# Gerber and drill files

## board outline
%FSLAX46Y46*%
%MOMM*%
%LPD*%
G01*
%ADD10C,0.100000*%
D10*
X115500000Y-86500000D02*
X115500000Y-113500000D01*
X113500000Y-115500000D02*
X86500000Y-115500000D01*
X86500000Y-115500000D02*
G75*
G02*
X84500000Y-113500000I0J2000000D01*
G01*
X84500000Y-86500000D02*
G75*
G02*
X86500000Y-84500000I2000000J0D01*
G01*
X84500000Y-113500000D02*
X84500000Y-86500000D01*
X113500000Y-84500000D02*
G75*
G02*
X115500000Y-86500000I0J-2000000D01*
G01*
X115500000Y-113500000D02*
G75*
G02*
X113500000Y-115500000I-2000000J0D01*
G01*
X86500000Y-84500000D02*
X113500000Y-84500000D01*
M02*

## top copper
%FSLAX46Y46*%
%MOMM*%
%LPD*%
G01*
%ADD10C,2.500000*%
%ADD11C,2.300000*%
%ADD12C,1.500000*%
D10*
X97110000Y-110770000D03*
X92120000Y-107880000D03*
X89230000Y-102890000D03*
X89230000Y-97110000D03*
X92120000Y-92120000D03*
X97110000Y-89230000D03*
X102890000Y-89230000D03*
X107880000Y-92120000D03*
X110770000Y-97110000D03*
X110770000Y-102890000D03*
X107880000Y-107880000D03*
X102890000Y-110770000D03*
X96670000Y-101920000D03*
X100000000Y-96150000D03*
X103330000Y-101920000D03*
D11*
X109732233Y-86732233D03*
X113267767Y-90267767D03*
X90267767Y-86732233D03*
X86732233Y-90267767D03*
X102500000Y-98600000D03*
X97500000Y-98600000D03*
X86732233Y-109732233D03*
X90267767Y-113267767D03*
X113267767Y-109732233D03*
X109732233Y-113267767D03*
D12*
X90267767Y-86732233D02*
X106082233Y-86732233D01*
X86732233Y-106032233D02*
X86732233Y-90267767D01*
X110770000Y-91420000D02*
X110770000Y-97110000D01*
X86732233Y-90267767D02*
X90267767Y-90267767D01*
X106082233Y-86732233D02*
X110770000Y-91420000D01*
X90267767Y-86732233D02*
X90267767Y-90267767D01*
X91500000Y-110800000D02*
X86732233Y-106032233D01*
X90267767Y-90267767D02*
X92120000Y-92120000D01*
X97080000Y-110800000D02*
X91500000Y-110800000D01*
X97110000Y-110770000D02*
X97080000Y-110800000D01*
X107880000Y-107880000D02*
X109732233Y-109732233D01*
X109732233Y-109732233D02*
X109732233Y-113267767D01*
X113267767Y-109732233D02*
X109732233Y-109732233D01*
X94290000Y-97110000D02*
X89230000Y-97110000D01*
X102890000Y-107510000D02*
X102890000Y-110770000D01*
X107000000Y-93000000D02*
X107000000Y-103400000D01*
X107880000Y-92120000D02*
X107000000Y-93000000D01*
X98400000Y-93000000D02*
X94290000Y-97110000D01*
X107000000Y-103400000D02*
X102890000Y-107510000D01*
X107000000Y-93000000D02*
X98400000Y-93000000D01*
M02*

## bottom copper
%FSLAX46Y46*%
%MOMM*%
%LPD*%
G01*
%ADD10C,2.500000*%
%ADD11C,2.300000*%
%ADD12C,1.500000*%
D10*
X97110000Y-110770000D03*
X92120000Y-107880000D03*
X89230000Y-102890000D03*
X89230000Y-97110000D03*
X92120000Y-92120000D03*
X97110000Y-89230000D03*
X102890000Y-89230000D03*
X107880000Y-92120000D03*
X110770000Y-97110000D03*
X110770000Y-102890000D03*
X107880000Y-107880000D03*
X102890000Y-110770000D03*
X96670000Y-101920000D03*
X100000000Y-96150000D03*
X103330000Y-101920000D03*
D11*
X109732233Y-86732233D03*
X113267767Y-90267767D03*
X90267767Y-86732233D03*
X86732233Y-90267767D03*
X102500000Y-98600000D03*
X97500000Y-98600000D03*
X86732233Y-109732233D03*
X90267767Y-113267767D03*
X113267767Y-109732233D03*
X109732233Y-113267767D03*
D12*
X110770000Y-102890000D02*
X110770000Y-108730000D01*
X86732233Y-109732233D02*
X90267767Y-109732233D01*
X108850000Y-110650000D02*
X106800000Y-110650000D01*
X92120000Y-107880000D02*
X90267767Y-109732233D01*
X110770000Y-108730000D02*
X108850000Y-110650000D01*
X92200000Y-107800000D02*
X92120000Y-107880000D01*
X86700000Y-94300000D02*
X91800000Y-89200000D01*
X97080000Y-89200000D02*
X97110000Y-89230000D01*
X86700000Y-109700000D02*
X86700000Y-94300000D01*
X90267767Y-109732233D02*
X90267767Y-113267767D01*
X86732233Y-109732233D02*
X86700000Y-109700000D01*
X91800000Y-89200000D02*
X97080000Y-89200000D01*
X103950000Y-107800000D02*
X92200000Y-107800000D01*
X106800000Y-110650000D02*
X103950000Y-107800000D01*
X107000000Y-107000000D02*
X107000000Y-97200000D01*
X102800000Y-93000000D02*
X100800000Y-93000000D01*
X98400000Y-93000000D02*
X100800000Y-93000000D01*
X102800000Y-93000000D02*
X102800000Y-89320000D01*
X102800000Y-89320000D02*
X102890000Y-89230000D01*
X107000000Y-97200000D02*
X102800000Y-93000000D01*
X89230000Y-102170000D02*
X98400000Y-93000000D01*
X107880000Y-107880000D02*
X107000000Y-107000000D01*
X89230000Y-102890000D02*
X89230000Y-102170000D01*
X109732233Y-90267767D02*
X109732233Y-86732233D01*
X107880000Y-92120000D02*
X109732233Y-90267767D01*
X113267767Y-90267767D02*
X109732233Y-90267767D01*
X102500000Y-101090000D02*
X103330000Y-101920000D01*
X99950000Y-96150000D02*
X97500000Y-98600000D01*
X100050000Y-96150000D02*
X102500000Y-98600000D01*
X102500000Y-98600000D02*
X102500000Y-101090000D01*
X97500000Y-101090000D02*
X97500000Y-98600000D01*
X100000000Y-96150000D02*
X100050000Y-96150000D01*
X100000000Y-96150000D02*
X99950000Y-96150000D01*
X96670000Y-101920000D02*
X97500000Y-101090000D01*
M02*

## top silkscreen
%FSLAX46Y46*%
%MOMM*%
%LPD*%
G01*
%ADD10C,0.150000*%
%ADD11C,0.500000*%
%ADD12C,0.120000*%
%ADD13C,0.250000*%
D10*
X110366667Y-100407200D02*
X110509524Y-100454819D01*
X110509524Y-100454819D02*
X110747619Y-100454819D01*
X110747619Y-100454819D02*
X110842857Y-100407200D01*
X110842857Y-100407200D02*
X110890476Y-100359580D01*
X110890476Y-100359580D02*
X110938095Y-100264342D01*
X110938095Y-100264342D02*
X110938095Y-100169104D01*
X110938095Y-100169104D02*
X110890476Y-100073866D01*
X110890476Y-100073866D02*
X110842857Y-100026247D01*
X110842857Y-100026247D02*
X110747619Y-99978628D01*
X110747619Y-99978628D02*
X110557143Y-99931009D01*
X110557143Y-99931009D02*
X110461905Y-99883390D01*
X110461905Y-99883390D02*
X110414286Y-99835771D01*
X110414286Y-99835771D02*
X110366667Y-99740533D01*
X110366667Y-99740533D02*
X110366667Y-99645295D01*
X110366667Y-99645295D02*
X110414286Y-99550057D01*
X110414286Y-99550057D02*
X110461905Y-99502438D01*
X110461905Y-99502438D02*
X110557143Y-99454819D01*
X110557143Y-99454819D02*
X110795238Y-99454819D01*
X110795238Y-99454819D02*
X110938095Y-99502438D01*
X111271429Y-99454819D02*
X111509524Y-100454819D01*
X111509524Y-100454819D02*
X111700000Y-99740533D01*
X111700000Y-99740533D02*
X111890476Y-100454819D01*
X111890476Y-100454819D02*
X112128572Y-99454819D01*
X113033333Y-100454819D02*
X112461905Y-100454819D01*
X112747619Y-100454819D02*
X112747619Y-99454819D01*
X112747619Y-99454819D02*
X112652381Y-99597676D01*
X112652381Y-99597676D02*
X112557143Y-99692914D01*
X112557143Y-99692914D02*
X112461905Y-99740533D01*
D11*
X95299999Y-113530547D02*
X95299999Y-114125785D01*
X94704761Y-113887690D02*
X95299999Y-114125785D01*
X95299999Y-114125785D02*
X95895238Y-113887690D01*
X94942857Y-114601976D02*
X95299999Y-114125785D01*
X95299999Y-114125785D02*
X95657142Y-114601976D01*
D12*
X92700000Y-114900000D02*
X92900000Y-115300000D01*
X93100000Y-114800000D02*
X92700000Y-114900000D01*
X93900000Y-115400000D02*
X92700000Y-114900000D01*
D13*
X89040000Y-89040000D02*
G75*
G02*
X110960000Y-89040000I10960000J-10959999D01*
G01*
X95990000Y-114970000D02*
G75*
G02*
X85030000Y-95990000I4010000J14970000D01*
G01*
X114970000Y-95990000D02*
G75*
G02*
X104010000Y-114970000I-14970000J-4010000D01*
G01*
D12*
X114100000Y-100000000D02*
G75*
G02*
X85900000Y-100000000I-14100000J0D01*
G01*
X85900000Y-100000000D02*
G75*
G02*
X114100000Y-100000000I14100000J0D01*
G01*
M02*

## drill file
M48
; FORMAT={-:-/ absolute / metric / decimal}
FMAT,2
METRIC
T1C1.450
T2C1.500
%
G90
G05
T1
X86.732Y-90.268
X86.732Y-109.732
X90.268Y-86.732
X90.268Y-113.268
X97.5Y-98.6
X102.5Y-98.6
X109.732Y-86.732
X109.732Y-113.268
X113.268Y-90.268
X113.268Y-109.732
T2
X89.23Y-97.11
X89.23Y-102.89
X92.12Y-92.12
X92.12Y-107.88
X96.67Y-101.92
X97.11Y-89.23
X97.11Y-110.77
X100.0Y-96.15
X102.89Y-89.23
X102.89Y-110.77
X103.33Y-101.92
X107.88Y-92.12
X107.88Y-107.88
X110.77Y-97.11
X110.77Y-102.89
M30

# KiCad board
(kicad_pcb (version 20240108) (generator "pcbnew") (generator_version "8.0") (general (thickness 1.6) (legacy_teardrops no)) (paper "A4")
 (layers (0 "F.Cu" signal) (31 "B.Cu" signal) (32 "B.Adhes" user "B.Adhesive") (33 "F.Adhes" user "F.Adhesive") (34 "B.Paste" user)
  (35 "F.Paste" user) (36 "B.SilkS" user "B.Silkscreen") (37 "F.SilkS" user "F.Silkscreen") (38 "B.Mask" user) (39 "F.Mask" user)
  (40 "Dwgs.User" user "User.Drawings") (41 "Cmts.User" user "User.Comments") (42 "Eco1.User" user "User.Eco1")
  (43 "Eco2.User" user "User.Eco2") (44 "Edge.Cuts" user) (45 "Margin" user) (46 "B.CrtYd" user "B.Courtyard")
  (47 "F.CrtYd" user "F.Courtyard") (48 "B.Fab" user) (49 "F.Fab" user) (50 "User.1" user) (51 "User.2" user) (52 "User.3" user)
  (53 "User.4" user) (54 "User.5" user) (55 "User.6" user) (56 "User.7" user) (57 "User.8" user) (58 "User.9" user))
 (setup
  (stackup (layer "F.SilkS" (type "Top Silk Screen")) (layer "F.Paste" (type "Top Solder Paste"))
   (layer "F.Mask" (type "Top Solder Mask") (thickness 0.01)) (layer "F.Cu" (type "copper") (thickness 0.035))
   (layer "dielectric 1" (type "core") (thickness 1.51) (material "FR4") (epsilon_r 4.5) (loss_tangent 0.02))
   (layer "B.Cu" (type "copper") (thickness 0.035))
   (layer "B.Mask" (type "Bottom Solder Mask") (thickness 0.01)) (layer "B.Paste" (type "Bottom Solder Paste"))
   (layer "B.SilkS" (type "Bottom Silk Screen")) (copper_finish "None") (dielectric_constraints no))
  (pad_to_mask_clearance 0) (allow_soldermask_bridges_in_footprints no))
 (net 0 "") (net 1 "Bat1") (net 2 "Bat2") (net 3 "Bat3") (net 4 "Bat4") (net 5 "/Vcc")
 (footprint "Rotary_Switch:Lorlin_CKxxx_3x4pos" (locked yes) (layer "F.Cu") (at 100 100)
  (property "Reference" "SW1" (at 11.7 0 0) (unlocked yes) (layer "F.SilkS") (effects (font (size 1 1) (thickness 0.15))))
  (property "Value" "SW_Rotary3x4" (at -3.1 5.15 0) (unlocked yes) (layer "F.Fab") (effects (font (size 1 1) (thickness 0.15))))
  (fp_line (start -7.3 14.9) (end -7.1 15.3) (stroke (width 0.12) (type solid)) (layer "F.SilkS"))
  (fp_line (start -6.9 14.8) (end -7.3 14.9) (stroke (width 0.12) (type solid)) (layer "F.SilkS"))
  (fp_line (start -6.1 15.4) (end -7.3 14.9) (stroke (width 0.12) (type solid)) (layer "F.SilkS"))
  (fp_arc (start -10.96 -10.96) (mid 0 -15.499781) (end 10.96 -10.96) (stroke (width 0.25) (type solid)) (layer "F.SilkS"))
  (fp_arc (start -4.01 14.97) (mid -13.420887 7.74989) (end -14.97 -4.01) (stroke (width 0.25) (type solid)) (layer "F.SilkS"))
  (fp_arc (start 14.97 -4.01) (mid 13.420887 7.74989) (end 4.01 14.97) (stroke (width 0.25) (type solid)) (layer "F.SilkS"))
  (fp_circle (center 0 0) (end 14.1 0) (stroke (width 0.12) (type solid)) (fill none) (layer "F.SilkS"))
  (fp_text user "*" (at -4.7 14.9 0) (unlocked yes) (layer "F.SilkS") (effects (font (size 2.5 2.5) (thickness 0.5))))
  (pad "1" thru_hole circle (at -2.89 10.77) (size 2.5 2.5) (drill 1.5) (layers "*.Cu" "*.Mask") (remove_unused_layers no) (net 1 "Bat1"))
  (pad "2" thru_hole circle (at -7.88 7.88) (size 2.5 2.5) (drill 1.5) (layers "*.Cu" "*.Mask") (remove_unused_layers no) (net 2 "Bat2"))
  (pad "3" thru_hole circle (at -10.77 2.89) (size 2.5 2.5) (drill 1.5) (layers "*.Cu" "*.Mask") (remove_unused_layers no) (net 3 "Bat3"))
  (pad "4" thru_hole circle (at -10.77 -2.89) (size 2.5 2.5) (drill 1.5) (layers "*.Cu" "*.Mask") (remove_unused_layers no) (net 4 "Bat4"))
  (pad "5" thru_hole circle (at -7.88 -7.88) (size 2.5 2.5) (drill 1.5) (layers "*.Cu" "*.Mask") (remove_unused_layers no) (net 1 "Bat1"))
  (pad "6" thru_hole circle (at -2.89 -10.77) (size 2.5 2.5) (drill 1.5) (layers "*.Cu" "*.Mask") (remove_unused_layers no) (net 2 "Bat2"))
  (pad "7" thru_hole circle (at 2.89 -10.77) (size 2.5 2.5) (drill 1.5) (layers "*.Cu" "*.Mask") (remove_unused_layers no) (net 3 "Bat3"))
  (pad "8" thru_hole circle (at 7.88 -7.88) (size 2.5 2.5) (drill 1.5) (layers "*.Cu" "*.Mask") (remove_unused_layers no) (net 4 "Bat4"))
  (pad "9" thru_hole circle (at 10.77 -2.89) (size 2.5 2.5) (drill 1.5) (layers "*.Cu" "*.Mask") (remove_unused_layers no) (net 1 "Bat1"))
  (pad "10" thru_hole circle (at 10.77 2.89) (size 2.5 2.5) (drill 1.5) (layers "*.Cu" "*.Mask") (remove_unused_layers no) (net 2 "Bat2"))
  (pad "11" thru_hole circle (at 7.88 7.88) (size 2.5 2.5) (drill 1.5) (layers "*.Cu" "*.Mask") (remove_unused_layers no) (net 3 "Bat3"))
  (pad "12" thru_hole circle (at 2.89 10.77) (size 2.5 2.5) (drill 1.5) (layers "*.Cu" "*.Mask") (remove_unused_layers no) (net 4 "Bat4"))
  (pad "13" thru_hole circle (at -3.33 1.92) (size 2.5 2.5) (drill 1.5) (layers "*.Cu" "*.Mask") (remove_unused_layers no) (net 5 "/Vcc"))
  (pad "14" thru_hole circle (at 0 -3.85) (size 2.5 2.5) (drill 1.5) (layers "*.Cu" "*.Mask") (remove_unused_layers no) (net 5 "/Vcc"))
  (pad "15" thru_hole circle (at 3.33 1.92) (size 2.5 2.5) (drill 1.5) (layers "*.Cu" "*.Mask") (remove_unused_layers no) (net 5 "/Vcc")))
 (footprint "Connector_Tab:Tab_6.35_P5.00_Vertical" (layer "B.Cu") (at 111.5 88.5 -45)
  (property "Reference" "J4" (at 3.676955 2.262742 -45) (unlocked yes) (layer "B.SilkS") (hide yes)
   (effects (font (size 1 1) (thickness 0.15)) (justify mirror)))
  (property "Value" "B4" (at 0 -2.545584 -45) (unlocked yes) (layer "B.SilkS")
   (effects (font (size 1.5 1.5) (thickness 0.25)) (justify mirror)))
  (pad "1" thru_hole circle (at -2.5 0 315) (size 2.3 2.3) (drill 1.45) (layers "*.Cu" "*.Mask") (remove_unused_layers no) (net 4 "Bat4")
   (clearance 0.3))
  (pad "1" thru_hole circle (at 2.5 0 315) (size 2.3 2.3) (drill 1.45) (layers "*.Cu" "*.Mask") (remove_unused_layers no) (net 4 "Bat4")
   (clearance 0.3)))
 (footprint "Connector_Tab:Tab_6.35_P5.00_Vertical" (layer "B.Cu") (at 88.5 88.5 -135)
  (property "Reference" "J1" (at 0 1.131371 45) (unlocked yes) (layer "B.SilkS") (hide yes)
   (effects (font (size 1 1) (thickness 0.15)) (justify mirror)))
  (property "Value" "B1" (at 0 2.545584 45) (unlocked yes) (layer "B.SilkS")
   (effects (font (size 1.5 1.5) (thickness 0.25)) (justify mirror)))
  (pad "1" thru_hole circle (at -2.5 0 225) (size 2.3 2.3) (drill 1.45) (layers "*.Cu" "*.Mask") (remove_unused_layers no) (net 1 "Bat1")
   (clearance 0.3))
  (pad "1" thru_hole circle (at 2.5 0 225) (size 2.3 2.3) (drill 1.45) (layers "*.Cu" "*.Mask") (remove_unused_layers no) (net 1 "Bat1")
   (clearance 0.3)))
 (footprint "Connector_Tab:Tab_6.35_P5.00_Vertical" (layer "B.Cu") (at 100 98.6 180)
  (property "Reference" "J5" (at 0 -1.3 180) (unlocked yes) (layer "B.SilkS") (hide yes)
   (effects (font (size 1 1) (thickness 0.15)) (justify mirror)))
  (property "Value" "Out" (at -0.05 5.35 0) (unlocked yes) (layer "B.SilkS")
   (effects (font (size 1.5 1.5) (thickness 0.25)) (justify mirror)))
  (pad "1" thru_hole circle (at -2.5 0 180) (size 2.3 2.3) (drill 1.45) (layers "*.Cu" "*.Mask") (remove_unused_layers no) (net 5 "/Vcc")
   (clearance 0.3))
  (pad "1" thru_hole circle (at 2.5 0 180) (size 2.3 2.3) (drill 1.45) (layers "*.Cu" "*.Mask") (remove_unused_layers no) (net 5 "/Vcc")
   (clearance 0.3)))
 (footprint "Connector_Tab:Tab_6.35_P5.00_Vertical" (layer "B.Cu") (at 88.5 111.5 -45)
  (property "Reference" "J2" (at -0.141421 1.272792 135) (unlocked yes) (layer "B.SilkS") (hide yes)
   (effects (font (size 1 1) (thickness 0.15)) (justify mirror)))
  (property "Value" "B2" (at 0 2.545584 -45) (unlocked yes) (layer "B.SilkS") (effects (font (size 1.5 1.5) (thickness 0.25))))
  (pad "1" thru_hole circle (at -2.5 0 315) (size 2.3 2.3) (drill 1.45) (layers "*.Cu" "*.Mask") (remove_unused_layers no) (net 2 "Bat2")
   (clearance 0.3))
  (pad "1" thru_hole circle (at 2.5 0 315) (size 2.3 2.3) (drill 1.45) (layers "*.Cu" "*.Mask") (remove_unused_layers no) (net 2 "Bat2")
   (clearance 0.3)))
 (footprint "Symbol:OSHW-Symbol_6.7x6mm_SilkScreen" (layer "B.Cu") (at 100 106 180)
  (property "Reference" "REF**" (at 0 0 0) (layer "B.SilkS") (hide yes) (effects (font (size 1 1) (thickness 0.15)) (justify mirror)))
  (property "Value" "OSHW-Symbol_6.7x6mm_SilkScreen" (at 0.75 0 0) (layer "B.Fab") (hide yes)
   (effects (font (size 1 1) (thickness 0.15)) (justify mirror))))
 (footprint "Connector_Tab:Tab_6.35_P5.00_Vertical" (layer "B.Cu") (at 111.5 111.5 -135)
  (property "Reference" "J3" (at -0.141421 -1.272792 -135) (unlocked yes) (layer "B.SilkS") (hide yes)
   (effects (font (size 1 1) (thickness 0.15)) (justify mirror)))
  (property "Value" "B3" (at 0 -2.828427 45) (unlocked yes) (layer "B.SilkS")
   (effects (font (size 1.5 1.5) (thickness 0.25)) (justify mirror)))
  (pad "1" thru_hole circle (at -2.5 0 225) (size 2.3 2.3) (drill 1.45) (layers "*.Cu" "*.Mask") (remove_unused_layers no) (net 3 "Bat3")
   (clearance 0.3))
  (pad "1" thru_hole circle (at 2.5 0 225) (size 2.3 2.3) (drill 1.45) (layers "*.Cu" "*.Mask") (remove_unused_layers no) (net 3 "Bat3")
   (clearance 0.3)))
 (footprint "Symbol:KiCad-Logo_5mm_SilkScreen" (layer "B.Cu") (at 107.167938 99.982906 -90)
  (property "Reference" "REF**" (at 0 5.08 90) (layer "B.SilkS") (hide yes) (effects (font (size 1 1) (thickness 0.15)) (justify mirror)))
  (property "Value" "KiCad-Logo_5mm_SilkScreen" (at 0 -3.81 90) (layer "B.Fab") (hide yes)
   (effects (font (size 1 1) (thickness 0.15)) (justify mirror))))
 (gr_line (start 115.5 86.5) (end 115.5 113.5) (stroke (width 0.1) (type solid)) (layer "Edge.Cuts"))
 (gr_line (start 113.5 115.5) (end 86.5 115.5) (stroke (width 0.1) (type solid)) (layer "Edge.Cuts"))
 (gr_arc (start 86.5 115.5) (mid 85.085786 114.914214) (end 84.5 113.5) (stroke (width 0.1) (type solid)) (layer "Edge.Cuts"))
 (gr_arc (start 84.5 86.5) (mid 85.085786 85.085786) (end 86.5 84.5) (stroke (width 0.1) (type solid)) (layer "Edge.Cuts"))
 (gr_line (start 84.5 113.5) (end 84.5 86.5) (stroke (width 0.1) (type solid)) (layer "Edge.Cuts"))
 (gr_arc (start 113.5 84.5) (mid 114.914214 85.085786) (end 115.5 86.5) (stroke (width 0.1) (type solid)) (layer "Edge.Cuts"))
 (gr_arc (start 115.5 113.5) (mid 114.914214 114.914214) (end 113.5 115.5) (stroke (width 0.1) (type solid)) (layer "Edge.Cuts"))
 (gr_line (start 86.5 84.5) (end 113.5 84.5) (stroke (width 0.1) (type solid)) (layer "Edge.Cuts"))
 (segment (start 90.267767 86.732233) (end 106.082233 86.732233) (width 1.5) (layer "F.Cu") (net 1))
 (segment (start 86.732233 106.032233) (end 86.732233 90.267767) (width 1.5) (layer "F.Cu") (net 1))
 (segment (start 110.77 91.42) (end 110.77 97.11) (width 1.5) (layer "F.Cu") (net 1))
 (segment (start 86.732233 90.267767) (end 90.267767 90.267767) (width 1.5) (layer "F.Cu") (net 1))
 (segment (start 106.082233 86.732233) (end 110.77 91.42) (width 1.5) (layer "F.Cu") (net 1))
 (segment (start 90.267767 86.732233) (end 90.267767 90.267767) (width 1.5) (layer "F.Cu") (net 1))
 (segment (start 91.5 110.8) (end 86.732233 106.032233) (width 1.5) (layer "F.Cu") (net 1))
 (segment (start 90.267767 90.267767) (end 92.12 92.12) (width 1.5) (layer "F.Cu") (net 1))
 (segment (start 97.08 110.8) (end 91.5 110.8) (width 1.5) (layer "F.Cu") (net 1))
 (segment (start 97.11 110.77) (end 97.08 110.8) (width 1.5) (layer "F.Cu") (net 1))
 (segment (start 110.77 102.89) (end 110.77 108.73) (width 1.5) (layer "B.Cu") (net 2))
 (segment (start 86.732233 109.732233) (end 90.267767 109.732233) (width 1.5) (layer "B.Cu") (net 2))
 (segment (start 108.85 110.65) (end 106.8 110.65) (width 1.5) (layer "B.Cu") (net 2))
 (segment (start 92.12 107.88) (end 90.267767 109.732233) (width 1.5) (layer "B.Cu") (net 2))
 (segment (start 110.77 108.73) (end 108.85 110.65) (width 1.5) (layer "B.Cu") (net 2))
 (segment (start 92.2 107.8) (end 92.12 107.88) (width 1.5) (layer "B.Cu") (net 2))
 (segment (start 86.7 94.3) (end 91.8 89.2) (width 1.5) (layer "B.Cu") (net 2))
 (segment (start 97.08 89.2) (end 97.11 89.23) (width 1.5) (layer "B.Cu") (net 2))
 (segment (start 86.7 109.7) (end 86.7 94.3) (width 1.5) (layer "B.Cu") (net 2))
 (segment (start 90.267767 109.732233) (end 90.267767 113.267767) (width 1.5) (layer "B.Cu") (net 2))
 (segment (start 86.732233 109.732233) (end 86.7 109.7) (width 1.5) (layer "B.Cu") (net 2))
 (segment (start 91.8 89.2) (end 97.08 89.2) (width 1.5) (layer "B.Cu") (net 2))
 (segment (start 103.95 107.8) (end 92.2 107.8) (width 1.5) (layer "B.Cu") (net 2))
 (segment (start 106.8 110.65) (end 103.95 107.8) (width 1.5) (layer "B.Cu") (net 2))
 (segment (start 107.88 107.88) (end 109.732233 109.732233) (width 1.5) (layer "F.Cu") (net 3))
 (segment (start 109.732233 109.732233) (end 109.732233 113.267767) (width 1.5) (layer "F.Cu") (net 3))
 (segment (start 113.267767 109.732233) (end 109.732233 109.732233) (width 1.5) (layer "F.Cu") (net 3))
 (segment (start 107 107) (end 107 97.2) (width 1.5) (layer "B.Cu") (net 3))
 (segment (start 102.8 93) (end 100.8 93) (width 1.5) (layer "B.Cu") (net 3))
 (segment (start 98.4 93) (end 100.8 93) (width 1.5) (layer "B.Cu") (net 3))
 (segment (start 102.8 93) (end 102.8 89.32) (width 1.5) (layer "B.Cu") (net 3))
 (segment (start 102.8 89.32) (end 102.89 89.23) (width 1.5) (layer "B.Cu") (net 3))
 (segment (start 107 97.2) (end 102.8 93) (width 1.5) (layer "B.Cu") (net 3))
 (segment (start 89.23 102.17) (end 98.4 93) (width 1.5) (layer "B.Cu") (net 3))
 (segment (start 107.88 107.88) (end 107 107) (width 1.5) (layer "B.Cu") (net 3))
 (segment (start 89.23 102.89) (end 89.23 102.17) (width 1.5) (layer "B.Cu") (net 3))
 (segment (start 94.29 97.11) (end 89.23 97.11) (width 1.5) (layer "F.Cu") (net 4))
 (segment (start 102.89 107.51) (end 102.89 110.77) (width 1.5) (layer "F.Cu") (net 4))
 (segment (start 107 93) (end 107 103.4) (width 1.5) (layer "F.Cu") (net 4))
 (segment (start 107.88 92.12) (end 107 93) (width 1.5) (layer "F.Cu") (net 4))
 (segment (start 98.4 93) (end 94.29 97.11) (width 1.5) (layer "F.Cu") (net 4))
 (segment (start 107 103.4) (end 102.89 107.51) (width 1.5) (layer "F.Cu") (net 4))
 (segment (start 107 93) (end 98.4 93) (width 1.5) (layer "F.Cu") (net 4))
 (segment (start 109.732233 90.267767) (end 109.732233 86.732233) (width 1.5) (layer "B.Cu") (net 4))
 (segment (start 107.88 92.12) (end 109.732233 90.267767) (width 1.5) (layer "B.Cu") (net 4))
 (segment (start 113.267767 90.267767) (end 109.732233 90.267767) (width 1.5) (layer "B.Cu") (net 4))
 (segment (start 102.5 101.09) (end 103.33 101.92) (width 1.5) (layer "B.Cu") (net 5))
 (segment (start 99.95 96.15) (end 97.5 98.6) (width 1.5) (layer "B.Cu") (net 5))
 (segment (start 100.05 96.15) (end 102.5 98.6) (width 1.5) (layer "B.Cu") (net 5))
 (segment (start 102.5 98.6) (end 102.5 101.09) (width 1.5) (layer "B.Cu") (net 5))
 (segment (start 97.5 101.09) (end 97.5 98.6) (width 1.5) (layer "B.Cu") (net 5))
 (segment (start 100 96.15) (end 100.05 96.15) (width 1.5) (layer "B.Cu") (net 5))
 (segment (start 100 96.15) (end 99.95 96.15) (width 1.5) (layer "B.Cu") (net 5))
 (segment (start 96.67 101.92) (end 97.5 101.09) (width 1.5) (layer "B.Cu") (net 5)))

